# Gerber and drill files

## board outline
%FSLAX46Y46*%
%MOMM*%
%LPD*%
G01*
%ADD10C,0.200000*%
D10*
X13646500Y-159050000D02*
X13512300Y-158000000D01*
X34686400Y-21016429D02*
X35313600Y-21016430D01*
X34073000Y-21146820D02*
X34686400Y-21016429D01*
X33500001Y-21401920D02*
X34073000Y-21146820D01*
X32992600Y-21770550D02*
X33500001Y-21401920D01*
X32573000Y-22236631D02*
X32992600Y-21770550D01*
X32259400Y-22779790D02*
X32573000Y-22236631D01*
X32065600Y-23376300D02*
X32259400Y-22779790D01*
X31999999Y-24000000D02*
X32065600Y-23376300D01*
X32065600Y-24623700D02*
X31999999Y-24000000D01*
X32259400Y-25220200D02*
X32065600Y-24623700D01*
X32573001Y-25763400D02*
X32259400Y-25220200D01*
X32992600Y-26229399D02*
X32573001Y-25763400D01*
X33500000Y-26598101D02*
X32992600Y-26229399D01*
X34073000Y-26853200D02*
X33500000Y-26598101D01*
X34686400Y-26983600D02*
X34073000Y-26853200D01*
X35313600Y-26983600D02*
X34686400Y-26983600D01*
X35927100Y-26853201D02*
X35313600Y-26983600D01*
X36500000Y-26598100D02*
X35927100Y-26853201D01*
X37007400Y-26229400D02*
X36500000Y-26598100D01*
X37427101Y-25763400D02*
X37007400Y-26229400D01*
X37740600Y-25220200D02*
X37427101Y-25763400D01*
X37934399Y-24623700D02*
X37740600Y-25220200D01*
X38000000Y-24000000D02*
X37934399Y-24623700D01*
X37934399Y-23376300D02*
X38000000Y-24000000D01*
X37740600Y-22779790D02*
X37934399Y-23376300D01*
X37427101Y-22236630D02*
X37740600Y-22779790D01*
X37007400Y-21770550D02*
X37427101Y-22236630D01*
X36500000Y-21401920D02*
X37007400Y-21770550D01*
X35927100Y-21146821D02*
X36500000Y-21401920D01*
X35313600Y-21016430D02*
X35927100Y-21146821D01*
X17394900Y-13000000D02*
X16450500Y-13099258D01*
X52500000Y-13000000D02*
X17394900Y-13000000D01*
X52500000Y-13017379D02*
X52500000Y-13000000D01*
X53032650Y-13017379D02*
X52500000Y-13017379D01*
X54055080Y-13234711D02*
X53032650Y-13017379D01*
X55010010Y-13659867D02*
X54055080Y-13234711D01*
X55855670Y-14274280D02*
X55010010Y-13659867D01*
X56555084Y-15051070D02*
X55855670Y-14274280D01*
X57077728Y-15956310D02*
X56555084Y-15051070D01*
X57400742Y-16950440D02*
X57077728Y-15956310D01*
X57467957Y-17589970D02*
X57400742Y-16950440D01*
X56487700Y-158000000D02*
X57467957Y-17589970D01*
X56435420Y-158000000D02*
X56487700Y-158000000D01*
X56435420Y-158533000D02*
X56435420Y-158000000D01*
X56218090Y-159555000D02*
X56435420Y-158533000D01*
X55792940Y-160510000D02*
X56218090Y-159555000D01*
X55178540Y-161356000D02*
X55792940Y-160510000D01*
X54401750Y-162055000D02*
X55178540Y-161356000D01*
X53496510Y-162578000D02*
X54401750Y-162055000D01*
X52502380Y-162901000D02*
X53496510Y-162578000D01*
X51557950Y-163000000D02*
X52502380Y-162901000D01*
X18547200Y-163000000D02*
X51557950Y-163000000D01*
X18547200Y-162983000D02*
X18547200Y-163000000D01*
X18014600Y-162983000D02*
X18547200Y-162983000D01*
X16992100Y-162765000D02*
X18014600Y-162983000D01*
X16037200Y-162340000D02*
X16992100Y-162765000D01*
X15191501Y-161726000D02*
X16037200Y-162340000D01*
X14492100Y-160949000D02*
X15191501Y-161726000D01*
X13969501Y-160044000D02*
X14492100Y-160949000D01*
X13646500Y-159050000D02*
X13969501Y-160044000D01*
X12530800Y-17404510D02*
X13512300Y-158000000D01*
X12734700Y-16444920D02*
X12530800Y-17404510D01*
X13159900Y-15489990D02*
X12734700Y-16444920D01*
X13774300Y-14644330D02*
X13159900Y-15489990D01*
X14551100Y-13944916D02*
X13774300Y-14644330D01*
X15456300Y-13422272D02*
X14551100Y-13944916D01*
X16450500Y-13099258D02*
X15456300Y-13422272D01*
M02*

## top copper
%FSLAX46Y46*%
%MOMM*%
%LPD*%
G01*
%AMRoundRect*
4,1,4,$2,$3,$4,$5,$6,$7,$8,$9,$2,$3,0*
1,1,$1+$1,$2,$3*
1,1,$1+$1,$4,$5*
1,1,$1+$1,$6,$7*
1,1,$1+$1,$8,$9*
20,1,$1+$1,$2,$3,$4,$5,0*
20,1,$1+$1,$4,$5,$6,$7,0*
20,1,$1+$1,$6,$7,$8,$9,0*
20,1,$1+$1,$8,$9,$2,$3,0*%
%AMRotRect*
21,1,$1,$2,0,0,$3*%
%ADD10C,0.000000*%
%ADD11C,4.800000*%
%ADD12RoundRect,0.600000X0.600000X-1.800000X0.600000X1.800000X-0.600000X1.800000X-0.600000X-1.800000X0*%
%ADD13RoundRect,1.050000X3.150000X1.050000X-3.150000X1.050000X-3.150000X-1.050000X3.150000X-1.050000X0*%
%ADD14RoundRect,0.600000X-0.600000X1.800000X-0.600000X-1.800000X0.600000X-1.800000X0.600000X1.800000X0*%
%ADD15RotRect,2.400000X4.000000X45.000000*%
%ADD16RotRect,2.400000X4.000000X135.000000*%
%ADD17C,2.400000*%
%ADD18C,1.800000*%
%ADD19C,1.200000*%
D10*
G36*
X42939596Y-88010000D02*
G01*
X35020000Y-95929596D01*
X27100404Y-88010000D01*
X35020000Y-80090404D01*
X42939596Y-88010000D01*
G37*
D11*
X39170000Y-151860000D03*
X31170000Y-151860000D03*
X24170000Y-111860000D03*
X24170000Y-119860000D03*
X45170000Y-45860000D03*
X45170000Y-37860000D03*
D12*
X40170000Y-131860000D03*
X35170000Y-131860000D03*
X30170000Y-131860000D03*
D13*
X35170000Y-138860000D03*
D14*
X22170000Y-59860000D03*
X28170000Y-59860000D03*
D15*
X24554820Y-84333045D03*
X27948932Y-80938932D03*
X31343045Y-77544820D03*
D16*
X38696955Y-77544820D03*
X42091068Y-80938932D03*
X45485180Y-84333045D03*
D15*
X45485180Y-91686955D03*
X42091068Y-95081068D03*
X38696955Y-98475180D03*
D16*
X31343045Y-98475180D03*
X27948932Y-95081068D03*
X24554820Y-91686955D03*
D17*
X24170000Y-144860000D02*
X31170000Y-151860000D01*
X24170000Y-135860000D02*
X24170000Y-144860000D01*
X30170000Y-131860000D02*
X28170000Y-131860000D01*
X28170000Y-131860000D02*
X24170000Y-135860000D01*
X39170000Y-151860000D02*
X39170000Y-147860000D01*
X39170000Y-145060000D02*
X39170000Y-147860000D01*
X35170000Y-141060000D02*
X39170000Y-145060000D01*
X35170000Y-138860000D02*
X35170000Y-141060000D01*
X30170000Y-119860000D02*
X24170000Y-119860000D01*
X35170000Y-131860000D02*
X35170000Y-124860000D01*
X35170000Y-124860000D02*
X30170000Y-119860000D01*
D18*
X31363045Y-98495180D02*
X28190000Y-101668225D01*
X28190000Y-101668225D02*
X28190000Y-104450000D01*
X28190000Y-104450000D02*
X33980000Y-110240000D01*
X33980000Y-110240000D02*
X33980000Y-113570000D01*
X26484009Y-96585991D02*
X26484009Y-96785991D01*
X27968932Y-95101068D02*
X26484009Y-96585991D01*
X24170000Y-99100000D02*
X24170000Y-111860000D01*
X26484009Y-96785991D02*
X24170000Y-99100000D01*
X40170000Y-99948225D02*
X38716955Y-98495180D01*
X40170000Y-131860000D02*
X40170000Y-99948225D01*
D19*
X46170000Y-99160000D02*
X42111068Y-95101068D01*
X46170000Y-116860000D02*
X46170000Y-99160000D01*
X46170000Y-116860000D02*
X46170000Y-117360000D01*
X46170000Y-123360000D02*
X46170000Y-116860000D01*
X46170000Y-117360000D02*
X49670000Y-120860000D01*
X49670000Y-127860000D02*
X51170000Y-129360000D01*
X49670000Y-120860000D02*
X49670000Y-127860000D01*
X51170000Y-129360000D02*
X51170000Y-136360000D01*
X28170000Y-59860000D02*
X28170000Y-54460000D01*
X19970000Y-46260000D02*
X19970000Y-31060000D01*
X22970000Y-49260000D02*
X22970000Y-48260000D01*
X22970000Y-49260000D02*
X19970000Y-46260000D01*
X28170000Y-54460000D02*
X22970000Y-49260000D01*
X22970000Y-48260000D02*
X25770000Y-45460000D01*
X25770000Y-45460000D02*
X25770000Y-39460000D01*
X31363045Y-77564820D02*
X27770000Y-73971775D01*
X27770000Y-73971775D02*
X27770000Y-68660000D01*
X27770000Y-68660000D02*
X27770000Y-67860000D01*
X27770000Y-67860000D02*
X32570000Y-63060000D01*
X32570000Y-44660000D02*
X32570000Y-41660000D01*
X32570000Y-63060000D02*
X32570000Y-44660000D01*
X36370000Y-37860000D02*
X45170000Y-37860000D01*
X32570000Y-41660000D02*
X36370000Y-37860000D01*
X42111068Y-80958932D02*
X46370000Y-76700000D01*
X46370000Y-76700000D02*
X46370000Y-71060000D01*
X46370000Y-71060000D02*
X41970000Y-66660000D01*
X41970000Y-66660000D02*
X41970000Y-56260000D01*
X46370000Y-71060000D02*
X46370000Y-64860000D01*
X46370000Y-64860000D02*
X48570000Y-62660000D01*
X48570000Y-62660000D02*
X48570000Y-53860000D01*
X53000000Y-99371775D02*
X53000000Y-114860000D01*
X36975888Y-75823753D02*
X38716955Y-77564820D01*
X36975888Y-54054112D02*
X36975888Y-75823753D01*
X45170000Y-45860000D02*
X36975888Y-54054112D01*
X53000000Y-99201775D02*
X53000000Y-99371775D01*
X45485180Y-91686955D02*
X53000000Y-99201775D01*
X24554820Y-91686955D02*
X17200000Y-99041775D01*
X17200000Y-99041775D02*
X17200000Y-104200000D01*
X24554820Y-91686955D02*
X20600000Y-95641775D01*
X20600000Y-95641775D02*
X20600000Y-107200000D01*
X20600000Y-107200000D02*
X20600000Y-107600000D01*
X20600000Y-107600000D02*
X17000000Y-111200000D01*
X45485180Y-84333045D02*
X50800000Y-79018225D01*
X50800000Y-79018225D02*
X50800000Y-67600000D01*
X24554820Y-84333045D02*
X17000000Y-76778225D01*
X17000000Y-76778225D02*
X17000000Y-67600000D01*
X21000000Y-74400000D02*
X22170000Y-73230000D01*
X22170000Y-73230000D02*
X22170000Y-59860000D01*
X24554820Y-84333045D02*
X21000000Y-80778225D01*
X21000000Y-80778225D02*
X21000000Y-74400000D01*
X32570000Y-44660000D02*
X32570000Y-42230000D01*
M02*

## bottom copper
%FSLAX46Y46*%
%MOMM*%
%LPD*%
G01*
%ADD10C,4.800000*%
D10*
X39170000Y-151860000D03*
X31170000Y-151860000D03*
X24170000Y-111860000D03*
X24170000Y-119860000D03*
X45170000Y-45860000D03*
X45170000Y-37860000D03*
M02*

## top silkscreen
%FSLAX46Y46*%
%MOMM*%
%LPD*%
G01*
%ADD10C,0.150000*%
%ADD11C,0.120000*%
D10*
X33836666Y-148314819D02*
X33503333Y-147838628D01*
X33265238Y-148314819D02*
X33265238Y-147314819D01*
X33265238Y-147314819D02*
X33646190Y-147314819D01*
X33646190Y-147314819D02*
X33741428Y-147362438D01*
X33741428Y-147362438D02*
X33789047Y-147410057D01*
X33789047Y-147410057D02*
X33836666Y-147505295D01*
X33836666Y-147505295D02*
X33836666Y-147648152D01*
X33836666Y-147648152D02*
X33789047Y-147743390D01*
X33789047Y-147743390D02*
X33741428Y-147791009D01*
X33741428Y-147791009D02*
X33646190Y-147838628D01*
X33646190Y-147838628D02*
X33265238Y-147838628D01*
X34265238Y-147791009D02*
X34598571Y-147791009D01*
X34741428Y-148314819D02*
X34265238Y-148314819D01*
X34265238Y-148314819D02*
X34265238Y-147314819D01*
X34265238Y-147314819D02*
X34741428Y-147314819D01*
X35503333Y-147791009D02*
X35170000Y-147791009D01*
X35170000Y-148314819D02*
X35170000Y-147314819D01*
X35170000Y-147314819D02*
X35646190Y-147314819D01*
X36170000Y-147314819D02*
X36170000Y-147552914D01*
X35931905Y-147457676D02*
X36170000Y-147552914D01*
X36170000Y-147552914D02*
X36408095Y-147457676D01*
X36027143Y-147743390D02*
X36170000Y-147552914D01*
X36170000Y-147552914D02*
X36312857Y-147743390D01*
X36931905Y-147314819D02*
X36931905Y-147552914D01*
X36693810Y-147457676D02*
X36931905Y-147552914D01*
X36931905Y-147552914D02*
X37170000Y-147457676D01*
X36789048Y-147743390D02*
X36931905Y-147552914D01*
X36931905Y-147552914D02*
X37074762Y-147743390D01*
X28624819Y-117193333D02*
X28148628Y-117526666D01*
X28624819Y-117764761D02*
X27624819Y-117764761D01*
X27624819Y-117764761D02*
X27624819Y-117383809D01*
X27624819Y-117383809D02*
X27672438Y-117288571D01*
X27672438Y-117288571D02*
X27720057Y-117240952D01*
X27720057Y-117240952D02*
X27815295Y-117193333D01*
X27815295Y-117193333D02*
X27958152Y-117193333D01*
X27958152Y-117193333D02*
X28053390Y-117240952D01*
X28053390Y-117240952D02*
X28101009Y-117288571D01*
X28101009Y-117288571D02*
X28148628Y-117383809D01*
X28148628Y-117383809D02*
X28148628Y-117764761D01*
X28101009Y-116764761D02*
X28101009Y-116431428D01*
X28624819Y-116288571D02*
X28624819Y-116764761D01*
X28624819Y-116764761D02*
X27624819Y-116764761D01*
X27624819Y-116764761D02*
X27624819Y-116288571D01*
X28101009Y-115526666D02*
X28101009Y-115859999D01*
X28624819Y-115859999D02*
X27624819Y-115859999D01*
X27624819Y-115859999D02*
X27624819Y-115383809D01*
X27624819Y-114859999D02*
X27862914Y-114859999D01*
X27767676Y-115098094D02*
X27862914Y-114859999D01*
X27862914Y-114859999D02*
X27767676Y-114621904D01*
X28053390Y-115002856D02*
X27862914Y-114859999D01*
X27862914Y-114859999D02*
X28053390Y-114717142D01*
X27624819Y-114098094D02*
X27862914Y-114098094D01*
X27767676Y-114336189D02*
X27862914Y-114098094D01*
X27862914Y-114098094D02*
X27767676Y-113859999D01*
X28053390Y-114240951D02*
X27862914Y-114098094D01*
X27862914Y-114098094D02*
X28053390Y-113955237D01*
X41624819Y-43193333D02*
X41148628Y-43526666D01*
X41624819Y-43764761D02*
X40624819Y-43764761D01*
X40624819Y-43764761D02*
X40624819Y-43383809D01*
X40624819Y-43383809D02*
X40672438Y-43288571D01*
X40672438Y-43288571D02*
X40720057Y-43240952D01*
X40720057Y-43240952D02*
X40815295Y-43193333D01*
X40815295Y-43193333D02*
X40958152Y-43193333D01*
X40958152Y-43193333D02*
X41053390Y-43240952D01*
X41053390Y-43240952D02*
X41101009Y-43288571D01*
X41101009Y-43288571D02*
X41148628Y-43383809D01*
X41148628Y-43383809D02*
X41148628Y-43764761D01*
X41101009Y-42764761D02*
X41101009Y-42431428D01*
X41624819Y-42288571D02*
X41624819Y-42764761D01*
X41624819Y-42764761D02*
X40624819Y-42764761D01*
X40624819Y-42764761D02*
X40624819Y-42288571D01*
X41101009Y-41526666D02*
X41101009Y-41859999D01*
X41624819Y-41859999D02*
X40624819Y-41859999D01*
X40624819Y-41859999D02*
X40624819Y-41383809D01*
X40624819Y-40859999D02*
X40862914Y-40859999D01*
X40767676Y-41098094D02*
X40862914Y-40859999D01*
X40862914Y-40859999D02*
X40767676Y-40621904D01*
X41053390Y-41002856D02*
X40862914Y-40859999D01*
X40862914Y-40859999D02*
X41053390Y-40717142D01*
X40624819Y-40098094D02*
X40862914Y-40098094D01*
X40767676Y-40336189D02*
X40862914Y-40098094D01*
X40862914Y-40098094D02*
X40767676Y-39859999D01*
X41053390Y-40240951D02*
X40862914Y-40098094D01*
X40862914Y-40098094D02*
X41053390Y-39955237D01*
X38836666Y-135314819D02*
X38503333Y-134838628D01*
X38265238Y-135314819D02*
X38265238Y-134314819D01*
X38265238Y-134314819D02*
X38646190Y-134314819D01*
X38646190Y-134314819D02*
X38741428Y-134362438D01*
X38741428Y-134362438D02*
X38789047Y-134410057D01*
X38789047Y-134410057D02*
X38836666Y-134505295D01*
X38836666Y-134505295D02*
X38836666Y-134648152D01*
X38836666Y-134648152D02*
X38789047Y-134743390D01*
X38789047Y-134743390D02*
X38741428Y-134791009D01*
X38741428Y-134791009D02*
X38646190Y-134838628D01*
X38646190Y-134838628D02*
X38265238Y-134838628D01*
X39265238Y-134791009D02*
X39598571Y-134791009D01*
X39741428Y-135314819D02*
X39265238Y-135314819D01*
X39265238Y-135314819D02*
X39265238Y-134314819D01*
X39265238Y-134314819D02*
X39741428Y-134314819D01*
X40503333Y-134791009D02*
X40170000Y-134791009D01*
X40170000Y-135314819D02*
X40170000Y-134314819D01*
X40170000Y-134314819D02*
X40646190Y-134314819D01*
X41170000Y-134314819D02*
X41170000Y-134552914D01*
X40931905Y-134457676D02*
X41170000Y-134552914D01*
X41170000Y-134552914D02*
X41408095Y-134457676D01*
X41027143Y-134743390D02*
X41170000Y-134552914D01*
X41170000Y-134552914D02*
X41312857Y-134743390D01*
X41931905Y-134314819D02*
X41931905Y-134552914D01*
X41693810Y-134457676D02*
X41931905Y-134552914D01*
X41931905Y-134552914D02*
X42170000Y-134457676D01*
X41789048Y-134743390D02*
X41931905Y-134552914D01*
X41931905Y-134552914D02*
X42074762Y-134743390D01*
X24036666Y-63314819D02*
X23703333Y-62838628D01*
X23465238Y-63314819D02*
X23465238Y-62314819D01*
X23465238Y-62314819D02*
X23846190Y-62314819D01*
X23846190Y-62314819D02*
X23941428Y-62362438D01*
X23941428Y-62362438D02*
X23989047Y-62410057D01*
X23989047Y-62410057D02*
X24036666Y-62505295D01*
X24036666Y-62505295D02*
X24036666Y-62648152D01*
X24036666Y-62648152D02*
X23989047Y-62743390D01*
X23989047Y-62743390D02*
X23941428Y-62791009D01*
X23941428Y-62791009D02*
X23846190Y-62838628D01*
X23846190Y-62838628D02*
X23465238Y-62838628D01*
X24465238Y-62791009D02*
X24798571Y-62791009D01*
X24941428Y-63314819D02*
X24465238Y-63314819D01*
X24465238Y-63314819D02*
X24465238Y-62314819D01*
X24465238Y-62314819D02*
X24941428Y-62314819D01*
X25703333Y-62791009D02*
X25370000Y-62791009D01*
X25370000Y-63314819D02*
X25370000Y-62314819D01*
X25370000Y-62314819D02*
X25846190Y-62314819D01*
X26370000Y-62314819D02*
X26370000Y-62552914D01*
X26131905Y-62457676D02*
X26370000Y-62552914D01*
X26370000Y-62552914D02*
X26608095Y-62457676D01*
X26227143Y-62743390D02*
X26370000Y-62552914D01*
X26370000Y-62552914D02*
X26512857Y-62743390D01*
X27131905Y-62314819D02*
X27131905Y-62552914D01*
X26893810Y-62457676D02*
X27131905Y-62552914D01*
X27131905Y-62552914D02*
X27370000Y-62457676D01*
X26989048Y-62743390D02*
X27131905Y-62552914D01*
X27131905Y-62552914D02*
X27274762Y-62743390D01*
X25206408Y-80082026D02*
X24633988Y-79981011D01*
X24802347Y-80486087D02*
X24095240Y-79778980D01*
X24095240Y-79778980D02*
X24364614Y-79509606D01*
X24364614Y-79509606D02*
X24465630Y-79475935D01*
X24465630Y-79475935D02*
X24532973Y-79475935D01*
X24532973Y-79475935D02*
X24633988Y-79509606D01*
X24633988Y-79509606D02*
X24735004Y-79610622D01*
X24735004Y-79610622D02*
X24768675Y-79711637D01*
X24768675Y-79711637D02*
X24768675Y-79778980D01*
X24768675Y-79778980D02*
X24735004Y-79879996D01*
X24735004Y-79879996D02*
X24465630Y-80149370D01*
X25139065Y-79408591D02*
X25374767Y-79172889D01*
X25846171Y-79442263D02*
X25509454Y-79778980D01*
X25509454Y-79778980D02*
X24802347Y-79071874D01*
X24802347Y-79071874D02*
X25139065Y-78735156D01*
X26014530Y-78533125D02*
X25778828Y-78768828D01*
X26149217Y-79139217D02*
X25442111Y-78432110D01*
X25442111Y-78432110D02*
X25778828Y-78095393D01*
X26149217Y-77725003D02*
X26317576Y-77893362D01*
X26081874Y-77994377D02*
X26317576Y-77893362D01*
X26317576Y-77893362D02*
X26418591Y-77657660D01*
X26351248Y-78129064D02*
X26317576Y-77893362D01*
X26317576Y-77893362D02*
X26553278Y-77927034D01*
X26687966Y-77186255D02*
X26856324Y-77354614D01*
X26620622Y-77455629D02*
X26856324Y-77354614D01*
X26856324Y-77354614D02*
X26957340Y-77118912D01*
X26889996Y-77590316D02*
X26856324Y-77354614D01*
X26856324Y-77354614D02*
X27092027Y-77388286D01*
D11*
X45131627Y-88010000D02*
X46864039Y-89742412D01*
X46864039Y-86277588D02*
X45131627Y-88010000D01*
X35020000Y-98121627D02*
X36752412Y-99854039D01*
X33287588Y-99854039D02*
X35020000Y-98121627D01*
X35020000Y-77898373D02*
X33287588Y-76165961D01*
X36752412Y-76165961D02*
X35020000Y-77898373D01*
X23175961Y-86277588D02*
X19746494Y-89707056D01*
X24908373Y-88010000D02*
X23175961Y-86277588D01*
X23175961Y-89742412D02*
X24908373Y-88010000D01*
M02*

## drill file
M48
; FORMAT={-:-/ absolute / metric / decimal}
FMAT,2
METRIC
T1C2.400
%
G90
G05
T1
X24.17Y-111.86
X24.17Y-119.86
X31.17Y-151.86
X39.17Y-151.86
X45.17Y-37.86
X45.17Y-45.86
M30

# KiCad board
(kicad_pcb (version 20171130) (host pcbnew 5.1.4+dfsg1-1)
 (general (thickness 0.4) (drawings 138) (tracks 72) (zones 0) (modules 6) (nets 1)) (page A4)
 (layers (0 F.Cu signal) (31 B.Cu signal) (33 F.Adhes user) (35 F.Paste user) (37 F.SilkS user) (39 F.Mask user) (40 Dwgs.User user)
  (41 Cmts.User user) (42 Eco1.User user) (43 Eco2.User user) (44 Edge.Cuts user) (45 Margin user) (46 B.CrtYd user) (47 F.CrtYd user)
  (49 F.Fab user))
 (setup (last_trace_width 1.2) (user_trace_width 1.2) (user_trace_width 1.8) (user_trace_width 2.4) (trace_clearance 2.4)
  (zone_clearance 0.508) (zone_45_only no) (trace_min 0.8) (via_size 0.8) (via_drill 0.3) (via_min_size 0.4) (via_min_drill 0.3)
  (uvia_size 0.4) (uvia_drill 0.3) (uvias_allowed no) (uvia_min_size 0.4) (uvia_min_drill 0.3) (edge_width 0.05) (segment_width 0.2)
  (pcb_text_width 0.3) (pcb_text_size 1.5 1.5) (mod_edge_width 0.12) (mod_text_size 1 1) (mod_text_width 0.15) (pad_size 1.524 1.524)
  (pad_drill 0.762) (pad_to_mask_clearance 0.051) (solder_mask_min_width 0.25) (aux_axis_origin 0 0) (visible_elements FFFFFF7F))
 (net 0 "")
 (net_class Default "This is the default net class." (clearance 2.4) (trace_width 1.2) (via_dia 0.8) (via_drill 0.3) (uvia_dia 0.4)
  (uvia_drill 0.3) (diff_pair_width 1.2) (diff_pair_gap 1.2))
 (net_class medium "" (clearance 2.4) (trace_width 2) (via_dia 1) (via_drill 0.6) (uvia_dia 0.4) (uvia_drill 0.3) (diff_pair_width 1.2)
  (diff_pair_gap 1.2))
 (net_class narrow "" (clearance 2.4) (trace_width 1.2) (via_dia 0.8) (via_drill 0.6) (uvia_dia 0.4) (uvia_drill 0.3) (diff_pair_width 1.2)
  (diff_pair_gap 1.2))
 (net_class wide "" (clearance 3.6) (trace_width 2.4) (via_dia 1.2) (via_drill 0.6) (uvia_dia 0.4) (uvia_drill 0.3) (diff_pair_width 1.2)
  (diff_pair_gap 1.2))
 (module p (layer F.Cu) (at 35.17 151.86)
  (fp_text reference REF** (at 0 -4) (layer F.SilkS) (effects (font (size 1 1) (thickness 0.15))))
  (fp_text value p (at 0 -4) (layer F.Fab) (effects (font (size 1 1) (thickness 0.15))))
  (pad 2 thru_hole circle (at 4 0) (size 4.8 4.8) (drill 2.4) (layers *.Cu *.Mask))
  (pad 1 thru_hole circle (at -4 0) (size 4.8 4.8) (drill 2.4) (layers *.Cu *.Mask)))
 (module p (layer F.Cu) (at 24.17 115.86 270)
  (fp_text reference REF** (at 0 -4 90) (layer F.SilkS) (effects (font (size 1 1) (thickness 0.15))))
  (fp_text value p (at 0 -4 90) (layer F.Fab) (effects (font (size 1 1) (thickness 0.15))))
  (pad 1 thru_hole circle (at -4 0 270) (size 4.8 4.8) (drill 2.4) (layers *.Cu *.Mask))
  (pad 2 thru_hole circle (at 4 0 270) (size 4.8 4.8) (drill 2.4) (layers *.Cu *.Mask)))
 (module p (layer F.Cu) (at 45.17 41.86 90)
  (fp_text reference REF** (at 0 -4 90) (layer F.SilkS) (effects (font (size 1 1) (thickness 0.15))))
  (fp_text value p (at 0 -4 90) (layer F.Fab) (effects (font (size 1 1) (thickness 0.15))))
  (pad 1 thru_hole circle (at -4 0 90) (size 4.8 4.8) (drill 2.4) (layers *.Cu *.Mask))
  (pad 2 thru_hole circle (at 4 0 90) (size 4.8 4.8) (drill 2.4) (layers *.Cu *.Mask)))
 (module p (layer F.Cu) (at 35.17 133.86 180)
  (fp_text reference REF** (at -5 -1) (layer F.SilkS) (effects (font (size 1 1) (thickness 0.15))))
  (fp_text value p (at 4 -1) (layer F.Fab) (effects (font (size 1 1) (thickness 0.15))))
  (pad 1 smd roundrect (at -5 2 90) (size 4.8 2.4) (layers F.Cu F.Paste F.Mask) (roundrect_rratio 0.25))
  (pad 2 smd roundrect (at 0 2 90) (size 4.8 2.4) (layers F.Cu F.Paste F.Mask) (roundrect_rratio 0.25))
  (pad 3 smd roundrect (at 5 2 90) (size 4.8 2.4) (layers F.Cu F.Paste F.Mask) (roundrect_rratio 0.25))
  (pad 4 smd roundrect (at 0 -5 180) (size 8.4 4.2) (layers F.Cu F.Paste F.Mask) (roundrect_rratio 0.25)))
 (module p (layer F.Cu) (at 25.17 59.86)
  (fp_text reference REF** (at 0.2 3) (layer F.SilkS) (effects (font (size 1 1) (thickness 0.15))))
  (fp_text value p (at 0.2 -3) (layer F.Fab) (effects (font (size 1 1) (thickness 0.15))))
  (pad 1 smd roundrect (at -3 0 270) (size 4.8 2.4) (layers F.Cu F.Paste F.Mask) (roundrect_rratio 0.25))
  (pad 2 smd roundrect (at 3 0 270) (size 4.8 2.4) (layers F.Cu F.Paste F.Mask) (roundrect_rratio 0.25)))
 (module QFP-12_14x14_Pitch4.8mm (layer F.Cu) (at 35.02 88.01 45)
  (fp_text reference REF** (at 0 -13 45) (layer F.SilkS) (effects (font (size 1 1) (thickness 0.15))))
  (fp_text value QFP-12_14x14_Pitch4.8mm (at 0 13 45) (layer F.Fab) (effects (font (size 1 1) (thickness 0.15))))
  (fp_poly (pts (xy -5.6 -5.6) (xy 5.6 -5.6) (xy 5.6 5.6) (xy -5.6 5.6)) (layer F.Cu) (width 0))
  (fp_line (start 7.15 7.15) (end 7.15 9.6) (layer F.SilkS) (width 0.12))
  (fp_line (start 9.6 7.15) (end 7.15 7.15) (layer F.SilkS) (width 0.12))
  (fp_line (start -7.15 7.15) (end -7.15 9.6) (layer F.SilkS) (width 0.12))
  (fp_line (start -9.6 7.15) (end -7.15 7.15) (layer F.SilkS) (width 0.12))
  (fp_line (start 7.15 -7.15) (end 7.15 -9.6) (layer F.SilkS) (width 0.12))
  (fp_line (start 9.6 -7.15) (end 7.15 -7.15) (layer F.SilkS) (width 0.12))
  (fp_line (start -7.15 -9.6) (end -12 -9.6) (layer F.SilkS) (width 0.12))
  (fp_line (start -7.15 -7.15) (end -7.15 -9.6) (layer F.SilkS) (width 0.12))
  (fp_line (start -9.6 -7.15) (end -7.15 -7.15) (layer F.SilkS) (width 0.12))
  (pad 12 smd rect (at -4.8 -10 45) (size 2.4 4) (layers F.Cu F.Paste F.Mask))
  (pad 11 smd rect (at 0 -10 45) (size 2.4 4) (layers F.Cu F.Paste F.Mask))
  (pad 10 smd rect (at 4.8 -10 45) (size 2.4 4) (layers F.Cu F.Paste F.Mask))
  (pad 9 smd rect (at 10 -4.8 135) (size 2.4 4) (layers F.Cu F.Paste F.Mask))
  (pad 8 smd rect (at 10 0 135) (size 2.4 4) (layers F.Cu F.Paste F.Mask))
  (pad 7 smd rect (at 10 4.8 135) (size 2.4 4) (layers F.Cu F.Paste F.Mask))
  (pad 6 smd rect (at 4.8 10 45) (size 2.4 4) (layers F.Cu F.Paste F.Mask))
  (pad 5 smd rect (at 0 10 45) (size 2.4 4) (layers F.Cu F.Paste F.Mask))
  (pad 4 smd rect (at -4.8 10 45) (size 2.4 4) (layers F.Cu F.Paste F.Mask))
  (pad 3 smd rect (at -10 4.8 135) (size 2.4 4) (layers F.Cu F.Paste F.Mask))
  (pad 2 smd rect (at -10 0 135) (size 2.4 4) (layers F.Cu F.Paste F.Mask))
  (pad 1 smd rect (at -10 -4.8 135) (size 2.4 4) (layers F.Cu F.Paste F.Mask)))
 (gr_line (start 13.6465 159.05) (end 13.5123 158) (layer Edge.Cuts) (width 0.2))
 (gr_line (start 34.6864 21.016429) (end 35.3136 21.01643) (layer Edge.Cuts) (width 0.2))
 (gr_line (start 34.073 21.14682) (end 34.6864 21.016429) (layer Edge.Cuts) (width 0.2))
 (gr_line (start 33.500001 21.40192) (end 34.073 21.14682) (layer Edge.Cuts) (width 0.2))
 (gr_line (start 32.9926 21.77055) (end 33.500001 21.40192) (layer Edge.Cuts) (width 0.2))
 (gr_line (start 32.573 22.236631) (end 32.9926 21.77055) (layer Edge.Cuts) (width 0.2))
 (gr_line (start 32.2594 22.77979) (end 32.573 22.236631) (layer Edge.Cuts) (width 0.2))
 (gr_line (start 32.0656 23.3763) (end 32.2594 22.77979) (layer Edge.Cuts) (width 0.2))
 (gr_line (start 31.999999 24) (end 32.0656 23.3763) (layer Edge.Cuts) (width 0.2))
 (gr_line (start 32.0656 24.6237) (end 31.999999 24) (layer Edge.Cuts) (width 0.2))
 (gr_line (start 32.2594 25.2202) (end 32.0656 24.6237) (layer Edge.Cuts) (width 0.2))
 (gr_line (start 32.573001 25.7634) (end 32.2594 25.2202) (layer Edge.Cuts) (width 0.2))
 (gr_line (start 32.9926 26.229399) (end 32.573001 25.7634) (layer Edge.Cuts) (width 0.2))
 (gr_line (start 33.5 26.598101) (end 32.9926 26.229399) (layer Edge.Cuts) (width 0.2))
 (gr_line (start 34.073 26.8532) (end 33.5 26.598101) (layer Edge.Cuts) (width 0.2))
 (gr_line (start 34.6864 26.9836) (end 34.073 26.8532) (layer Edge.Cuts) (width 0.2))
 (gr_line (start 35.3136 26.9836) (end 34.6864 26.9836) (layer Edge.Cuts) (width 0.2))
 (gr_line (start 35.9271 26.853201) (end 35.3136 26.9836) (layer Edge.Cuts) (width 0.2))
 (gr_line (start 36.5 26.5981) (end 35.9271 26.853201) (layer Edge.Cuts) (width 0.2))
 (gr_line (start 37.0074 26.2294) (end 36.5 26.5981) (layer Edge.Cuts) (width 0.2))
 (gr_line (start 37.427101 25.7634) (end 37.0074 26.2294) (layer Edge.Cuts) (width 0.2))
 (gr_line (start 37.7406 25.2202) (end 37.427101 25.7634) (layer Edge.Cuts) (width 0.2))
 (gr_line (start 37.934399 24.6237) (end 37.7406 25.2202) (layer Edge.Cuts) (width 0.2))
 (gr_line (start 38 24) (end 37.934399 24.6237) (layer Edge.Cuts) (width 0.2))
 (gr_line (start 37.934399 23.3763) (end 38 24) (layer Edge.Cuts) (width 0.2))
 (gr_line (start 37.7406 22.77979) (end 37.934399 23.3763) (layer Edge.Cuts) (width 0.2))
 (gr_line (start 37.427101 22.23663) (end 37.7406 22.77979) (layer Edge.Cuts) (width 0.2))
 (gr_line (start 37.0074 21.77055) (end 37.427101 22.23663) (layer Edge.Cuts) (width 0.2))
 (gr_line (start 36.5 21.40192) (end 37.0074 21.77055) (layer Edge.Cuts) (width 0.2))
 (gr_line (start 35.9271 21.146821) (end 36.5 21.40192) (layer Edge.Cuts) (width 0.2))
 (gr_line (start 35.3136 21.01643) (end 35.9271 21.146821) (layer Edge.Cuts) (width 0.2))
 (gr_line (start 17.3949 13) (end 16.4505 13.099258) (layer Edge.Cuts) (width 0.2))
 (gr_line (start 52.5 13) (end 17.3949 13) (layer Edge.Cuts) (width 0.2))
 (gr_line (start 52.5 13.017379) (end 52.5 13) (layer Edge.Cuts) (width 0.2))
 (gr_line (start 53.03265 13.017379) (end 52.5 13.017379) (layer Edge.Cuts) (width 0.2))
 (gr_line (start 54.05508 13.234711) (end 53.03265 13.017379) (layer Edge.Cuts) (width 0.2))
 (gr_line (start 55.01001 13.659867) (end 54.05508 13.234711) (layer Edge.Cuts) (width 0.2))
 (gr_line (start 55.85567 14.27428) (end 55.01001 13.659867) (layer Edge.Cuts) (width 0.2))
 (gr_line (start 56.555084 15.05107) (end 55.85567 14.27428) (layer Edge.Cuts) (width 0.2))
 (gr_line (start 57.077728 15.95631) (end 56.555084 15.05107) (layer Edge.Cuts) (width 0.2))
 (gr_line (start 57.400742 16.95044) (end 57.077728 15.95631) (layer Edge.Cuts) (width 0.2))
 (gr_line (start 57.467957 17.58997) (end 57.400742 16.95044) (layer Edge.Cuts) (width 0.2))
 (gr_line (start 56.4877 158) (end 57.467957 17.58997) (layer Edge.Cuts) (width 0.2))
 (gr_line (start 56.43542 158) (end 56.4877 158) (layer Edge.Cuts) (width 0.2))
 (gr_line (start 56.43542 158.533) (end 56.43542 158) (layer Edge.Cuts) (width 0.2))
 (gr_line (start 56.21809 159.555) (end 56.43542 158.533) (layer Edge.Cuts) (width 0.2))
 (gr_line (start 55.79294 160.51) (end 56.21809 159.555) (layer Edge.Cuts) (width 0.2))
 (gr_line (start 55.17854 161.356) (end 55.79294 160.51) (layer Edge.Cuts) (width 0.2))
 (gr_line (start 54.40175 162.055) (end 55.17854 161.356) (layer Edge.Cuts) (width 0.2))
 (gr_line (start 53.49651 162.578) (end 54.40175 162.055) (layer Edge.Cuts) (width 0.2))
 (gr_line (start 52.50238 162.901) (end 53.49651 162.578) (layer Edge.Cuts) (width 0.2))
 (gr_line (start 51.55795 163) (end 52.50238 162.901) (layer Edge.Cuts) (width 0.2))
 (gr_line (start 18.5472 163) (end 51.55795 163) (layer Edge.Cuts) (width 0.2))
 (gr_line (start 18.5472 162.983) (end 18.5472 163) (layer Edge.Cuts) (width 0.2))
 (gr_line (start 18.0146 162.983) (end 18.5472 162.983) (layer Edge.Cuts) (width 0.2))
 (gr_line (start 16.9921 162.765) (end 18.0146 162.983) (layer Edge.Cuts) (width 0.2))
 (gr_line (start 16.0372 162.34) (end 16.9921 162.765) (layer Edge.Cuts) (width 0.2))
 (gr_line (start 15.191501 161.726) (end 16.0372 162.34) (layer Edge.Cuts) (width 0.2))
 (gr_line (start 14.4921 160.949) (end 15.191501 161.726) (layer Edge.Cuts) (width 0.2))
 (gr_line (start 13.969501 160.044) (end 14.4921 160.949) (layer Edge.Cuts) (width 0.2))
 (gr_line (start 13.6465 159.05) (end 13.969501 160.044) (layer Edge.Cuts) (width 0.2))
 (gr_line (start 12.5308 17.40451) (end 13.5123 158) (layer Edge.Cuts) (width 0.2))
 (gr_line (start 12.7347 16.44492) (end 12.5308 17.40451) (layer Edge.Cuts) (width 0.2))
 (gr_line (start 13.1599 15.48999) (end 12.7347 16.44492) (layer Edge.Cuts) (width 0.2))
 (gr_line (start 13.7743 14.64433) (end 13.1599 15.48999) (layer Edge.Cuts) (width 0.2))
 (gr_line (start 14.5511 13.944916) (end 13.7743 14.64433) (layer Edge.Cuts) (width 0.2))
 (gr_line (start 15.4563 13.422272) (end 14.5511 13.944916) (layer Edge.Cuts) (width 0.2))
 (gr_line (start 16.4505 13.099258) (end 15.4563 13.422272) (layer Edge.Cuts) (width 0.2))
 (segment (start 24.17 144.86) (end 31.17 151.86) (width 2.4) (layer F.Cu) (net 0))
 (segment (start 24.17 135.86) (end 24.17 144.86) (width 2.4) (layer F.Cu) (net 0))
 (segment (start 30.17 131.86) (end 28.17 131.86) (width 2.4) (layer F.Cu) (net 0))
 (segment (start 28.17 131.86) (end 24.17 135.86) (width 2.4) (layer F.Cu) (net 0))
 (segment (start 39.17 151.86) (end 39.17 147.86) (width 2.4) (layer F.Cu) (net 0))
 (segment (start 39.17 145.06) (end 39.17 147.86) (width 2.4) (layer F.Cu) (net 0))
 (segment (start 35.17 141.06) (end 39.17 145.06) (width 2.4) (layer F.Cu) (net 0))
 (segment (start 35.17 138.86) (end 35.17 141.06) (width 2.4) (layer F.Cu) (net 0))
 (segment (start 30.17 119.86) (end 24.17 119.86) (width 2.4) (layer F.Cu) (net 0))
 (segment (start 35.17 131.86) (end 35.17 124.86) (width 2.4) (layer F.Cu) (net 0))
 (segment (start 35.17 124.86) (end 30.17 119.86) (width 2.4) (layer F.Cu) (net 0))
 (segment (start 31.363045 98.49518) (end 28.19 101.668225) (width 1.8) (layer F.Cu) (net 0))
 (segment (start 28.19 101.668225) (end 28.19 104.45) (width 1.8) (layer F.Cu) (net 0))
 (segment (start 28.19 104.45) (end 33.98 110.24) (width 1.8) (layer F.Cu) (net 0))
 (segment (start 33.98 110.24) (end 33.98 113.57) (width 1.8) (layer F.Cu) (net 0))
 (segment (start 26.484009 96.585991) (end 26.484009 96.785991) (width 1.8) (layer F.Cu) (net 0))
 (segment (start 27.968932 95.101068) (end 26.484009 96.585991) (width 1.8) (layer F.Cu) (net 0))
 (segment (start 24.17 99.1) (end 24.17 111.86) (width 1.8) (layer F.Cu) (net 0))
 (segment (start 26.484009 96.785991) (end 24.17 99.1) (width 1.8) (layer F.Cu) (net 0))
 (segment (start 40.17 99.948225) (end 38.716955 98.49518) (width 1.8) (layer F.Cu) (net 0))
 (segment (start 40.17 131.86) (end 40.17 99.948225) (width 1.8) (layer F.Cu) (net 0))
 (segment (start 46.17 99.16) (end 42.111068 95.101068) (width 1.2) (layer F.Cu) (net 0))
 (segment (start 46.17 116.86) (end 46.17 99.16) (width 1.2) (layer F.Cu) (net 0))
 (segment (start 46.17 116.86) (end 46.17 117.36) (width 1.2) (layer F.Cu) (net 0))
 (segment (start 46.17 123.36) (end 46.17 116.86) (width 1.2) (layer F.Cu) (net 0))
 (segment (start 46.17 117.36) (end 49.67 120.86) (width 1.2) (layer F.Cu) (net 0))
 (segment (start 49.67 127.86) (end 51.17 129.36) (width 1.2) (layer F.Cu) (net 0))
 (segment (start 49.67 120.86) (end 49.67 127.86) (width 1.2) (layer F.Cu) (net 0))
 (segment (start 51.17 129.36) (end 51.17 136.36) (width 1.2) (layer F.Cu) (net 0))
 (segment (start 28.17 59.86) (end 28.17 54.46) (width 1.2) (layer F.Cu) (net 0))
 (segment (start 19.97 46.26) (end 19.97 31.06) (width 1.2) (layer F.Cu) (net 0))
 (segment (start 22.97 49.26) (end 22.97 48.26) (width 1.2) (layer F.Cu) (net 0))
 (segment (start 22.97 49.26) (end 19.97 46.26) (width 1.2) (layer F.Cu) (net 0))
 (segment (start 28.17 54.46) (end 22.97 49.26) (width 1.2) (layer F.Cu) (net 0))
 (segment (start 22.97 48.26) (end 25.77 45.46) (width 1.2) (layer F.Cu) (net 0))
 (segment (start 25.77 45.46) (end 25.77 39.46) (width 1.2) (layer F.Cu) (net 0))
 (segment (start 31.363045 77.56482) (end 27.77 73.971775) (width 1.2) (layer F.Cu) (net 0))
 (segment (start 27.77 73.971775) (end 27.77 68.66) (width 1.2) (layer F.Cu) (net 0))
 (segment (start 27.77 68.66) (end 27.77 67.86) (width 1.2) (layer F.Cu) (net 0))
 (segment (start 27.77 67.86) (end 32.57 63.06) (width 1.2) (layer F.Cu) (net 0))
 (segment (start 32.57 44.66) (end 32.57 41.66) (width 1.2) (layer F.Cu) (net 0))
 (segment (start 32.57 63.06) (end 32.57 44.66) (width 1.2) (layer F.Cu) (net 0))
 (segment (start 36.37 37.86) (end 45.17 37.86) (width 1.2) (layer F.Cu) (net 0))
 (segment (start 32.57 41.66) (end 36.37 37.86) (width 1.2) (layer F.Cu) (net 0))
 (segment (start 42.111068 80.958932) (end 46.37 76.7) (width 1.2) (layer F.Cu) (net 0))
 (segment (start 46.37 76.7) (end 46.37 71.06) (width 1.2) (layer F.Cu) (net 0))
 (segment (start 46.37 71.06) (end 41.97 66.66) (width 1.2) (layer F.Cu) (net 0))
 (segment (start 41.97 66.66) (end 41.97 56.26) (width 1.2) (layer F.Cu) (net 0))
 (segment (start 46.37 71.06) (end 46.37 64.86) (width 1.2) (layer F.Cu) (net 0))
 (segment (start 46.37 64.86) (end 48.57 62.66) (width 1.2) (layer F.Cu) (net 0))
 (segment (start 48.57 62.66) (end 48.57 53.86) (width 1.2) (layer F.Cu) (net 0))
 (segment (start 53 99.371775) (end 53 114.86) (width 1.2) (layer F.Cu) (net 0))
 (segment (start 36.975888 75.823753) (end 38.716955 77.56482) (width 1.2) (layer F.Cu) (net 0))
 (segment (start 36.975888 54.054112) (end 36.975888 75.823753) (width 1.2) (layer F.Cu) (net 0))
 (segment (start 45.17 45.86) (end 36.975888 54.054112) (width 1.2) (layer F.Cu) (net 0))
 (segment (start 53 99.201775) (end 53 99.371775) (width 1.2) (layer F.Cu) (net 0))
 (segment (start 45.48518 91.686955) (end 53 99.201775) (width 1.2) (layer F.Cu) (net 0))
 (segment (start 24.55482 91.686955) (end 17.2 99.041775) (width 1.2) (layer F.Cu) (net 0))
 (segment (start 17.2 99.041775) (end 17.2 104.2) (width 1.2) (layer F.Cu) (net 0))
 (segment (start 24.55482 91.686955) (end 20.6 95.641775) (width 1.2) (layer F.Cu) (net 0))
 (segment (start 20.6 95.641775) (end 20.6 107.2) (width 1.2) (layer F.Cu) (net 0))
 (segment (start 20.6 107.2) (end 20.6 107.6) (width 1.2) (layer F.Cu) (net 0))
 (segment (start 20.6 107.6) (end 17 111.2) (width 1.2) (layer F.Cu) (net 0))
 (segment (start 45.48518 84.333045) (end 50.8 79.018225) (width 1.2) (layer F.Cu) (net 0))
 (segment (start 50.8 79.018225) (end 50.8 67.6) (width 1.2) (layer F.Cu) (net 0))
 (segment (start 24.55482 84.333045) (end 17 76.778225) (width 1.2) (layer F.Cu) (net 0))
 (segment (start 17 76.778225) (end 17 67.6) (width 1.2) (layer F.Cu) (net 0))
 (segment (start 21 74.4) (end 22.17 73.23) (width 1.2) (layer F.Cu) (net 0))
 (segment (start 22.17 73.23) (end 22.17 59.86) (width 1.2) (layer F.Cu) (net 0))
 (segment (start 24.55482 84.333045) (end 21 80.778225) (width 1.2) (layer F.Cu) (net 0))
 (segment (start 21 80.778225) (end 21 74.4) (width 1.2) (layer F.Cu) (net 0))
 (segment (start 32.57 44.66) (end 32.57 42.23) (width 1.2) (layer F.Cu) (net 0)))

